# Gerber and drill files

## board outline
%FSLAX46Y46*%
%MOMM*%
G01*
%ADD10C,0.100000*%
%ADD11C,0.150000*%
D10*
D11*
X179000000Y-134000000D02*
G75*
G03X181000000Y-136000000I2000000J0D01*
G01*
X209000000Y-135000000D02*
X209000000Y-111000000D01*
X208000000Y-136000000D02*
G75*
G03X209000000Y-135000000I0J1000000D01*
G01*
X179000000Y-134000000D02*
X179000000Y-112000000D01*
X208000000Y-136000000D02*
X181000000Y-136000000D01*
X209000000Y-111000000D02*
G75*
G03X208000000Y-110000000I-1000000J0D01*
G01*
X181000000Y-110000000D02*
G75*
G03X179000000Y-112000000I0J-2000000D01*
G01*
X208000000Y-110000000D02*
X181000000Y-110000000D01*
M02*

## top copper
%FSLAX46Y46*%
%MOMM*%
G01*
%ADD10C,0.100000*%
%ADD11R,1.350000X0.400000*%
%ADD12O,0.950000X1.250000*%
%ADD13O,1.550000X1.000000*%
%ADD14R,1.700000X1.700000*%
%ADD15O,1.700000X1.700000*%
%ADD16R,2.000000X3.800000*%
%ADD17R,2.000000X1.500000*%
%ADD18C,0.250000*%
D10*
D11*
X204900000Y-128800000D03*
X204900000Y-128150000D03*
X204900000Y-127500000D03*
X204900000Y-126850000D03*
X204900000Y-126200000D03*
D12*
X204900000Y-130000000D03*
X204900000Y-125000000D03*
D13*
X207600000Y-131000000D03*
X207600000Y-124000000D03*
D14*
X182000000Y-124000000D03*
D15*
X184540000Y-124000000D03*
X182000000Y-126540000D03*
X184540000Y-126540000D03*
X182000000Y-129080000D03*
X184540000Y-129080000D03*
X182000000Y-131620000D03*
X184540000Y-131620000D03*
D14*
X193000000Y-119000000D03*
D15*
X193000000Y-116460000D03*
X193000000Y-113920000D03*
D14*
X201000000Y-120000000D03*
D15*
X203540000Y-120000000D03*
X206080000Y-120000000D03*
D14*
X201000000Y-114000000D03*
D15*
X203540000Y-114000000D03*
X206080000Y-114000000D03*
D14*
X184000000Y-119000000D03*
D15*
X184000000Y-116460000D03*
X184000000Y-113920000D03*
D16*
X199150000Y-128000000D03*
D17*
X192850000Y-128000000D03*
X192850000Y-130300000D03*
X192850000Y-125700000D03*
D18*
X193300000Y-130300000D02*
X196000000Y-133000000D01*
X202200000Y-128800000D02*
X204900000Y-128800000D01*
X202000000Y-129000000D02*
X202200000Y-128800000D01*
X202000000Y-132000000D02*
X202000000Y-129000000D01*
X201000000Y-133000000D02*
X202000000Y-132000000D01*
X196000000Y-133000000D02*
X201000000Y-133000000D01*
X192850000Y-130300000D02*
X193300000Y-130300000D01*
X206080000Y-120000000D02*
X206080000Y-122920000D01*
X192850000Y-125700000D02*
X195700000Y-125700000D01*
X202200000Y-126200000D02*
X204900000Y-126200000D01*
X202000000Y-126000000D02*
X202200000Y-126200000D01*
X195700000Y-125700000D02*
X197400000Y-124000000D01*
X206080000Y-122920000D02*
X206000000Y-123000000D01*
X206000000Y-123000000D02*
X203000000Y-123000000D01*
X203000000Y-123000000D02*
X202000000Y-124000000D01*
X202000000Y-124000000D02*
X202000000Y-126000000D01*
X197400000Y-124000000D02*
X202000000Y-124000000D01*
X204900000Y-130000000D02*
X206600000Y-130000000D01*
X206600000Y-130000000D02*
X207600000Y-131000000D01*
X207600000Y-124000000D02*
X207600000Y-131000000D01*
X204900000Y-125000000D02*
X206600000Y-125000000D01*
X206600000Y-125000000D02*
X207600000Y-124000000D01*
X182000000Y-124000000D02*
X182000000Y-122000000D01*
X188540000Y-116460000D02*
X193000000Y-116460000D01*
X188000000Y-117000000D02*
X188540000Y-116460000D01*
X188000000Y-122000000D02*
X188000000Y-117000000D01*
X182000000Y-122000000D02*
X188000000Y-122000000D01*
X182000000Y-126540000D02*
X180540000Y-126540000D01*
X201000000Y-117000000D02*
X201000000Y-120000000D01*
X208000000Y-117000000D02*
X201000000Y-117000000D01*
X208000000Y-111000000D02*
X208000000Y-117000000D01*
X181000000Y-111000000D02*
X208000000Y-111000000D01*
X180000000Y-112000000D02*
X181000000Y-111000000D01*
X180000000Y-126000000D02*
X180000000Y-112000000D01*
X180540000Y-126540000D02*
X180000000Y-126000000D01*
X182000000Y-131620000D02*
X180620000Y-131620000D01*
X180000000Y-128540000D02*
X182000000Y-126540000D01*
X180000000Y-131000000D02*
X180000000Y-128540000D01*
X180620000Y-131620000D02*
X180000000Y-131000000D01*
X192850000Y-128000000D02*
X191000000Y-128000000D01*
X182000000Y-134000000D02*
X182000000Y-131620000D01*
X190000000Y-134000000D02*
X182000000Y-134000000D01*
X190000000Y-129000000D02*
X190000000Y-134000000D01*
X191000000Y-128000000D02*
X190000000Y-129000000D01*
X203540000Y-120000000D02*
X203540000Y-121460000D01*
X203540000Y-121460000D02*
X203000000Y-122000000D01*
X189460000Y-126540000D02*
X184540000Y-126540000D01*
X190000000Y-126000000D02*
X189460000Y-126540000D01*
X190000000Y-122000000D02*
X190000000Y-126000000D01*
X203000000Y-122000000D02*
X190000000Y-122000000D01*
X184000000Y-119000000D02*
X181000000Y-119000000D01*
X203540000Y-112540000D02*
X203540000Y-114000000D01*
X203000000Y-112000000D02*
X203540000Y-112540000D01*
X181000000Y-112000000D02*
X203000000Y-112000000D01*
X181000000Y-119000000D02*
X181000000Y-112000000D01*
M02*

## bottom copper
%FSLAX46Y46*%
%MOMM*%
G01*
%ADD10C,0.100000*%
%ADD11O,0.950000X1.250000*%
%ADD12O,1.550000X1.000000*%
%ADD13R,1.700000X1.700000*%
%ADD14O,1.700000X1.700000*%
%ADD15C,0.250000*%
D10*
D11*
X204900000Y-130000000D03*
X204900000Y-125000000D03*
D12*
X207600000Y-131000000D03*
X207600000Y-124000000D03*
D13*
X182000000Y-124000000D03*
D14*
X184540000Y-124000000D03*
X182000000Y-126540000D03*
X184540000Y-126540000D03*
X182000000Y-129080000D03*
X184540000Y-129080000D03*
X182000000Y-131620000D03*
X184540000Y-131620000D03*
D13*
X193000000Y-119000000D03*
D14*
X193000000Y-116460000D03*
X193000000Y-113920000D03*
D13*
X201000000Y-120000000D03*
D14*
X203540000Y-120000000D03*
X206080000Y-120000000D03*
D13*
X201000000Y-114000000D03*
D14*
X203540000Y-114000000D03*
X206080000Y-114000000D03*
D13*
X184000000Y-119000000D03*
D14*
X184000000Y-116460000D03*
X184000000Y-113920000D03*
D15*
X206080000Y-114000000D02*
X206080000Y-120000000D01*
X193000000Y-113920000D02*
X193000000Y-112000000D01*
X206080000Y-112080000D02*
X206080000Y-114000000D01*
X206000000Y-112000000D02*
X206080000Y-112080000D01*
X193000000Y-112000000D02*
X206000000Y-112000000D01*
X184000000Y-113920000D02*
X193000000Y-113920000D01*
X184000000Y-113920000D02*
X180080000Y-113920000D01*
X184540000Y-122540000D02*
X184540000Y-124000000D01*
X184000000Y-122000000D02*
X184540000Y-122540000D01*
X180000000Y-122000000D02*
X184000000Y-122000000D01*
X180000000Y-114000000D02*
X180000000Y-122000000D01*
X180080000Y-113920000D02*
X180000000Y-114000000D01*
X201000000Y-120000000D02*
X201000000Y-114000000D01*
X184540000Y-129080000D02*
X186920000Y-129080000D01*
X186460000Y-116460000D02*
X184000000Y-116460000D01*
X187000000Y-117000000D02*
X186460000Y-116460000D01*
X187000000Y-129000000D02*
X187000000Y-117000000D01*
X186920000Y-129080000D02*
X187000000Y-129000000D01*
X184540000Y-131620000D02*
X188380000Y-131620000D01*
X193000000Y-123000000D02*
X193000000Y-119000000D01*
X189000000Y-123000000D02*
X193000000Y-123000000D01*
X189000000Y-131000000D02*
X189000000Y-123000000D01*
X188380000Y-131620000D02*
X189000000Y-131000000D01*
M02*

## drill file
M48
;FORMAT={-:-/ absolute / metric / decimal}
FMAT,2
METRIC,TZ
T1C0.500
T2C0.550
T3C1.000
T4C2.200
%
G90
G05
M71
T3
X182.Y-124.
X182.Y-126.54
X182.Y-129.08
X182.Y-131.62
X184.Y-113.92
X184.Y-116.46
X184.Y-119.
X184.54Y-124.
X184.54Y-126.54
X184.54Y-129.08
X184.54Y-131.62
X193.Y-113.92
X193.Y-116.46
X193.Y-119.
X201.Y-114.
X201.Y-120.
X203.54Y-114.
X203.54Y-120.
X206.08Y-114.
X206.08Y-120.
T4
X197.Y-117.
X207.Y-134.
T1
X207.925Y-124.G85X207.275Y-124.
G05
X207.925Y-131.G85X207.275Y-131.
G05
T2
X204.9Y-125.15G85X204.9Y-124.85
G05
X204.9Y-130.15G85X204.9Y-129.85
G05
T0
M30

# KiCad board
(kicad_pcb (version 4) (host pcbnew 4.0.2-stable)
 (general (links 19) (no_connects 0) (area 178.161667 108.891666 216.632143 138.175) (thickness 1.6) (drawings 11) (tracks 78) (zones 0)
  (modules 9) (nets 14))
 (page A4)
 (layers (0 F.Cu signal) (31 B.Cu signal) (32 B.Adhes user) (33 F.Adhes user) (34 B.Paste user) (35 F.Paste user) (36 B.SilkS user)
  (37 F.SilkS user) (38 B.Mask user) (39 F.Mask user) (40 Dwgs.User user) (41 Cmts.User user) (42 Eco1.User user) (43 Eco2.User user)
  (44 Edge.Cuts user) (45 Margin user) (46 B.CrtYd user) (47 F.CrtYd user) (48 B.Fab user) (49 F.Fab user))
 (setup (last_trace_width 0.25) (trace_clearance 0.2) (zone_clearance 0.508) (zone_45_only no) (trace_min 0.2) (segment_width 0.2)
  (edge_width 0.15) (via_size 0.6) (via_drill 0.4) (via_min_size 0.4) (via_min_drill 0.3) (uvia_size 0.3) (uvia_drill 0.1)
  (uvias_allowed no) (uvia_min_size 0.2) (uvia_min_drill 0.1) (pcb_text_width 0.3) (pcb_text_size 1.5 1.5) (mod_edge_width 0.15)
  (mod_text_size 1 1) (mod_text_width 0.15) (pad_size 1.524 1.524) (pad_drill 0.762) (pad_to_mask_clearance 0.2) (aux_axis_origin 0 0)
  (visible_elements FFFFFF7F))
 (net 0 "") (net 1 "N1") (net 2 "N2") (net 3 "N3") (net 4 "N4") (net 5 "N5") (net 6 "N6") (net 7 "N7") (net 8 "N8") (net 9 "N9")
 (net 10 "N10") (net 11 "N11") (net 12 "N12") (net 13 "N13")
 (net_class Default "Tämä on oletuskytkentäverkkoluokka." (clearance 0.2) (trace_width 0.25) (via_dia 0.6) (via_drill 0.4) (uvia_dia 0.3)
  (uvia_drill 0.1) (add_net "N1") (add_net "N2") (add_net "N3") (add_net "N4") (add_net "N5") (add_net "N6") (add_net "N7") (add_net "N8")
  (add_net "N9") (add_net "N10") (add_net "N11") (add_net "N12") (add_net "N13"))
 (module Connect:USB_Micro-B (layer F.Cu) (at 206.25 127.5 90)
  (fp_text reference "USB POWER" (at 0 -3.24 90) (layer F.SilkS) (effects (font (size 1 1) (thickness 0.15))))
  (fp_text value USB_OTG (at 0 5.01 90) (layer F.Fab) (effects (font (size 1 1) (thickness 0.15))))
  (pad 1 smd rect (at -1.3 -1.35 180) (size 1.35 0.4) (layers F.Cu F.Paste F.Mask) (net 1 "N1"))
  (pad 2 smd rect (at -0.65 -1.35 180) (size 1.35 0.4) (layers F.Cu F.Paste F.Mask) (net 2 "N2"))
  (pad 3 smd rect (at 0 -1.35 180) (size 1.35 0.4) (layers F.Cu F.Paste F.Mask) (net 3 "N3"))
  (pad 4 smd rect (at 0.65 -1.35 180) (size 1.35 0.4) (layers F.Cu F.Paste F.Mask) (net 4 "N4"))
  (pad 5 smd rect (at 1.3 -1.35 180) (size 1.35 0.4) (layers F.Cu F.Paste F.Mask) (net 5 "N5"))
  (pad 6 thru_hole oval (at -2.5 -1.35 180) (size 0.95 1.25) (drill oval 0.55 0.85) (layers *.Cu *.Mask) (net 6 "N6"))
  (pad 6 thru_hole oval (at 2.5 -1.35 180) (size 0.95 1.25) (drill oval 0.55 0.85) (layers *.Cu *.Mask) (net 6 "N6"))
  (pad 6 thru_hole oval (at -3.5 1.35 180) (size 1.55 1) (drill oval 1.15 0.5) (layers *.Cu *.Mask) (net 6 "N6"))
  (pad 6 thru_hole oval (at 3.5 1.35 180) (size 1.55 1) (drill oval 1.15 0.5) (layers *.Cu *.Mask) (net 6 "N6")))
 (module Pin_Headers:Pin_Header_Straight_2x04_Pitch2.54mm (layer F.Cu) (at 182 124)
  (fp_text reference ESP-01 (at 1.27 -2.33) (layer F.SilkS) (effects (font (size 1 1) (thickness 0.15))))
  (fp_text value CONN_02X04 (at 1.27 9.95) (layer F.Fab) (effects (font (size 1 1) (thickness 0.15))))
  (pad 1 thru_hole rect (at 0 0) (size 1.7 1.7) (drill 1) (layers *.Cu *.Mask) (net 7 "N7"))
  (pad 2 thru_hole oval (at 2.54 0) (size 1.7 1.7) (drill 1) (layers *.Cu *.Mask) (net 5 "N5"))
  (pad 3 thru_hole oval (at 0 2.54) (size 1.7 1.7) (drill 1) (layers *.Cu *.Mask) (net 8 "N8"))
  (pad 4 thru_hole oval (at 2.54 2.54) (size 1.7 1.7) (drill 1) (layers *.Cu *.Mask) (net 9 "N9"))
  (pad 5 thru_hole oval (at 0 5.08) (size 1.7 1.7) (drill 1) (layers *.Cu *.Mask) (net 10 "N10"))
  (pad 6 thru_hole oval (at 2.54 5.08) (size 1.7 1.7) (drill 1) (layers *.Cu *.Mask) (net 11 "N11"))
  (pad 7 thru_hole oval (at 0 7.62) (size 1.7 1.7) (drill 1) (layers *.Cu *.Mask) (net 8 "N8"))
  (pad 8 thru_hole oval (at 2.54 7.62) (size 1.7 1.7) (drill 1) (layers *.Cu *.Mask) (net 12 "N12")))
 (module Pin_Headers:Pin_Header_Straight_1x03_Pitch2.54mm (layer F.Cu) (at 193 119 180)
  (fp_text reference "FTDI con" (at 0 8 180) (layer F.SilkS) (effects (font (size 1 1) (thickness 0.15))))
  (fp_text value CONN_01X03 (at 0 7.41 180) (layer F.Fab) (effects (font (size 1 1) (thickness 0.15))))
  (pad 1 thru_hole rect (at 0 0 180) (size 1.7 1.7) (drill 1) (layers *.Cu *.Mask) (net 12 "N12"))
  (pad 2 thru_hole oval (at 0 2.54 180) (size 1.7 1.7) (drill 1) (layers *.Cu *.Mask) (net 7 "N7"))
  (pad 3 thru_hole oval (at 0 5.08 180) (size 1.7 1.7) (drill 1) (layers *.Cu *.Mask) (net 5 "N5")))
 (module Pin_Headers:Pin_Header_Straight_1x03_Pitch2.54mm (layer F.Cu) (at 201 120 90)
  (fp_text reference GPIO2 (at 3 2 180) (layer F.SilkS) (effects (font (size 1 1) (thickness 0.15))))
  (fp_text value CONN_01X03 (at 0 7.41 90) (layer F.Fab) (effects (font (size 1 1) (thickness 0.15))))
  (pad 1 thru_hole rect (at 0 0 90) (size 1.7 1.7) (drill 1) (layers *.Cu *.Mask) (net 8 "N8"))
  (pad 2 thru_hole oval (at 0 2.54 90) (size 1.7 1.7) (drill 1) (layers *.Cu *.Mask) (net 9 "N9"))
  (pad 3 thru_hole oval (at 0 5.08 90) (size 1.7 1.7) (drill 1) (layers *.Cu *.Mask) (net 5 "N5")))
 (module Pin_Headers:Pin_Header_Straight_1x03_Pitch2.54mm (layer F.Cu) (at 201 114 90)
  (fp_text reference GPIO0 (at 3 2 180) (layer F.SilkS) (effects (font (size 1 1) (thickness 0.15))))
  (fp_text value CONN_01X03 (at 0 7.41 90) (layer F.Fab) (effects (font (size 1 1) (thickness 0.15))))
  (pad 1 thru_hole rect (at 0 0 90) (size 1.7 1.7) (drill 1) (layers *.Cu *.Mask) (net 8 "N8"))
  (pad 2 thru_hole oval (at 0 2.54 90) (size 1.7 1.7) (drill 1) (layers *.Cu *.Mask) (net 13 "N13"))
  (pad 3 thru_hole oval (at 0 5.08 90) (size 1.7 1.7) (drill 1) (layers *.Cu *.Mask) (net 5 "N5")))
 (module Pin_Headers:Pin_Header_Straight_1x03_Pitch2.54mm (layer F.Cu) (at 184 119 180)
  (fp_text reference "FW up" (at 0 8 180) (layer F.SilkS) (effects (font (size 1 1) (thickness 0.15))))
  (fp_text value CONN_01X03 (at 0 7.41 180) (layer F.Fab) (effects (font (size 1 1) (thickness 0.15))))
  (pad 1 thru_hole rect (at 0 0 180) (size 1.7 1.7) (drill 1) (layers *.Cu *.Mask) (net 13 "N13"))
  (pad 2 thru_hole oval (at 0 2.54 180) (size 1.7 1.7) (drill 1) (layers *.Cu *.Mask) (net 11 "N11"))
  (pad 3 thru_hole oval (at 0 5.08 180) (size 1.7 1.7) (drill 1) (layers *.Cu *.Mask) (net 5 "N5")))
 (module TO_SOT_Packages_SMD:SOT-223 (layer F.Cu) (at 196 128)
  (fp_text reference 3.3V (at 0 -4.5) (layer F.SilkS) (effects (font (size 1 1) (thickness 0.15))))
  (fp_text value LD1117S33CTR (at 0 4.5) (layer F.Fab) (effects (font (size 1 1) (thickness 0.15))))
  (pad 4 smd rect (at 3.15 0) (size 2 3.8) (layers F.Cu F.Paste F.Mask))
  (pad 2 smd rect (at -3.15 0) (size 2 1.5) (layers F.Cu F.Paste F.Mask) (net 8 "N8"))
  (pad 3 smd rect (at -3.15 2.3) (size 2 1.5) (layers F.Cu F.Paste F.Mask) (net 1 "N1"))
  (pad 1 smd rect (at -3.15 -2.3) (size 2 1.5) (layers F.Cu F.Paste F.Mask) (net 5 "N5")))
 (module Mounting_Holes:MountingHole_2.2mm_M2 (layer F.Cu) (at 197 117)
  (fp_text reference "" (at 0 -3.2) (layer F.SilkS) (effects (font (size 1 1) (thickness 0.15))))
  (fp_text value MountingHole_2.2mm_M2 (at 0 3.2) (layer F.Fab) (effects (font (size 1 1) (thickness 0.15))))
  (pad 1 np_thru_hole circle (at 0 0) (size 2.2 2.2) (drill 2.2) (layers *.Cu *.Mask)))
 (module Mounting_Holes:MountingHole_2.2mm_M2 (layer F.Cu) (at 207 134)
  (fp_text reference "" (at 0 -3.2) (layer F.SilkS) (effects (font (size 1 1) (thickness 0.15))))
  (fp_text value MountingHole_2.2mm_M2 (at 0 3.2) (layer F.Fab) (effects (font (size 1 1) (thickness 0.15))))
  (pad 1 np_thru_hole circle (at 0 0) (size 2.2 2.2) (drill 2.2) (layers *.Cu *.Mask)))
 (gr_arc (start 181 134) (end 181 136) (angle 90) (layer Edge.Cuts) (width 0.15))
 (gr_line (start 209 135) (end 209 111) (angle 90) (layer Edge.Cuts) (width 0.15))
 (gr_arc (start 208 135) (end 209 135) (angle 90) (layer Edge.Cuts) (width 0.15))
 (gr_line (start 179 134) (end 179 112) (angle 90) (layer Edge.Cuts) (width 0.15))
 (gr_line (start 208 136) (end 181 136) (angle 90) (layer Edge.Cuts) (width 0.15))
 (gr_arc (start 208 111) (end 208 110) (angle 90) (layer Edge.Cuts) (width 0.15))
 (gr_arc (start 181 112) (end 179 112) (angle 90) (layer Edge.Cuts) (width 0.15))
 (gr_line (start 208 110) (end 181 110) (angle 90) (layer Edge.Cuts) (width 0.15))
 (segment (start 193.3 130.3) (end 196 133) (width 0.25) (layer F.Cu) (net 1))
 (segment (start 202.2 128.8) (end 204.9 128.8) (width 0.25) (layer F.Cu) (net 1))
 (segment (start 202 129) (end 202.2 128.8) (width 0.25) (layer F.Cu) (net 1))
 (segment (start 202 132) (end 202 129) (width 0.25) (layer F.Cu) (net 1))
 (segment (start 201 133) (end 202 132) (width 0.25) (layer F.Cu) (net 1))
 (segment (start 196 133) (end 201 133) (width 0.25) (layer F.Cu) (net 1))
 (segment (start 192.85 130.3) (end 193.3 130.3) (width 0.25) (layer F.Cu) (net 1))
 (segment (start 206.08 114) (end 206.08 120) (width 0.25) (layer B.Cu) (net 5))
 (segment (start 193 113.92) (end 193 112) (width 0.25) (layer B.Cu) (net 5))
 (segment (start 206.08 112.08) (end 206.08 114) (width 0.25) (layer B.Cu) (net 5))
 (segment (start 206 112) (end 206.08 112.08) (width 0.25) (layer B.Cu) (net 5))
 (segment (start 193 112) (end 206 112) (width 0.25) (layer B.Cu) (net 5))
 (segment (start 184 113.92) (end 193 113.92) (width 0.25) (layer B.Cu) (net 5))
 (segment (start 184 113.92) (end 180.08 113.92) (width 0.25) (layer B.Cu) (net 5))
 (segment (start 184.54 122.54) (end 184.54 124) (width 0.25) (layer B.Cu) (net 5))
 (segment (start 184 122) (end 184.54 122.54) (width 0.25) (layer B.Cu) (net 5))
 (segment (start 180 122) (end 184 122) (width 0.25) (layer B.Cu) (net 5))
 (segment (start 180 114) (end 180 122) (width 0.25) (layer B.Cu) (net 5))
 (segment (start 180.08 113.92) (end 180 114) (width 0.25) (layer B.Cu) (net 5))
 (segment (start 206.08 120) (end 206.08 122.92) (width 0.25) (layer F.Cu) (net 5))
 (segment (start 192.85 125.7) (end 195.7 125.7) (width 0.25) (layer F.Cu) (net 5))
 (segment (start 202.2 126.2) (end 204.9 126.2) (width 0.25) (layer F.Cu) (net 5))
 (segment (start 202 126) (end 202.2 126.2) (width 0.25) (layer F.Cu) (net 5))
 (segment (start 195.7 125.7) (end 197.4 124) (width 0.25) (layer F.Cu) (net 5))
 (segment (start 206.08 122.92) (end 206 123) (width 0.25) (layer F.Cu) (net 5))
 (segment (start 206 123) (end 203 123) (width 0.25) (layer F.Cu) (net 5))
 (segment (start 203 123) (end 202 124) (width 0.25) (layer F.Cu) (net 5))
 (segment (start 202 124) (end 202 126) (width 0.25) (layer F.Cu) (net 5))
 (segment (start 197.4 124) (end 202 124) (width 0.25) (layer F.Cu) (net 5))
 (segment (start 204.9 130) (end 206.6 130) (width 0.25) (layer F.Cu) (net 6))
 (segment (start 206.6 130) (end 207.6 131) (width 0.25) (layer F.Cu) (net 6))
 (segment (start 207.6 124) (end 207.6 131) (width 0.25) (layer F.Cu) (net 6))
 (segment (start 204.9 125) (end 206.6 125) (width 0.25) (layer F.Cu) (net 6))
 (segment (start 206.6 125) (end 207.6 124) (width 0.25) (layer F.Cu) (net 6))
 (segment (start 182 124) (end 182 122) (width 0.25) (layer F.Cu) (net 7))
 (segment (start 188.54 116.46) (end 193 116.46) (width 0.25) (layer F.Cu) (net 7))
 (segment (start 188 117) (end 188.54 116.46) (width 0.25) (layer F.Cu) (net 7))
 (segment (start 188 122) (end 188 117) (width 0.25) (layer F.Cu) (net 7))
 (segment (start 182 122) (end 188 122) (width 0.25) (layer F.Cu) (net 7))
 (segment (start 201 120) (end 201 114) (width 0.25) (layer B.Cu) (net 8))
 (segment (start 182 126.54) (end 180.54 126.54) (width 0.25) (layer F.Cu) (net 8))
 (segment (start 201 117) (end 201 120) (width 0.25) (layer F.Cu) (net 8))
 (segment (start 208 117) (end 201 117) (width 0.25) (layer F.Cu) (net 8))
 (segment (start 208 111) (end 208 117) (width 0.25) (layer F.Cu) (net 8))
 (segment (start 181 111) (end 208 111) (width 0.25) (layer F.Cu) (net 8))
 (segment (start 180 112) (end 181 111) (width 0.25) (layer F.Cu) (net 8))
 (segment (start 180 126) (end 180 112) (width 0.25) (layer F.Cu) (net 8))
 (segment (start 180.54 126.54) (end 180 126) (width 0.25) (layer F.Cu) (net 8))
 (segment (start 182 131.62) (end 180.62 131.62) (width 0.25) (layer F.Cu) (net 8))
 (segment (start 180 128.54) (end 182 126.54) (width 0.25) (layer F.Cu) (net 8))
 (segment (start 180 131) (end 180 128.54) (width 0.25) (layer F.Cu) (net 8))
 (segment (start 180.62 131.62) (end 180 131) (width 0.25) (layer F.Cu) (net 8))
 (segment (start 192.85 128) (end 191 128) (width 0.25) (layer F.Cu) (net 8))
 (segment (start 182 134) (end 182 131.62) (width 0.25) (layer F.Cu) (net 8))
 (segment (start 190 134) (end 182 134) (width 0.25) (layer F.Cu) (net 8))
 (segment (start 190 129) (end 190 134) (width 0.25) (layer F.Cu) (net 8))
 (segment (start 191 128) (end 190 129) (width 0.25) (layer F.Cu) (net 8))
 (segment (start 203.54 120) (end 203.54 121.46) (width 0.25) (layer F.Cu) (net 9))
 (segment (start 203.54 121.46) (end 203 122) (width 0.25) (layer F.Cu) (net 9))
 (segment (start 189.46 126.54) (end 184.54 126.54) (width 0.25) (layer F.Cu) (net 9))
 (segment (start 190 126) (end 189.46 126.54) (width 0.25) (layer F.Cu) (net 9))
 (segment (start 190 122) (end 190 126) (width 0.25) (layer F.Cu) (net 9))
 (segment (start 203 122) (end 190 122) (width 0.25) (layer F.Cu) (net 9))
 (segment (start 184.54 129.08) (end 186.92 129.08) (width 0.25) (layer B.Cu) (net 11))
 (segment (start 186.46 116.46) (end 184 116.46) (width 0.25) (layer B.Cu) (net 11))
 (segment (start 187 117) (end 186.46 116.46) (width 0.25) (layer B.Cu) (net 11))
 (segment (start 187 129) (end 187 117) (width 0.25) (layer B.Cu) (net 11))
 (segment (start 186.92 129.08) (end 187 129) (width 0.25) (layer B.Cu) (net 11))
 (segment (start 184.54 131.62) (end 188.38 131.62) (width 0.25) (layer B.Cu) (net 12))
 (segment (start 193 123) (end 193 119) (width 0.25) (layer B.Cu) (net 12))
 (segment (start 189 123) (end 193 123) (width 0.25) (layer B.Cu) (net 12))
 (segment (start 189 131) (end 189 123) (width 0.25) (layer B.Cu) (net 12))
 (segment (start 188.38 131.62) (end 189 131) (width 0.25) (layer B.Cu) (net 12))
 (segment (start 184 119) (end 181 119) (width 0.25) (layer F.Cu) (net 13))
 (segment (start 203.54 112.54) (end 203.54 114) (width 0.25) (layer F.Cu) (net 13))
 (segment (start 203 112) (end 203.54 112.54) (width 0.25) (layer F.Cu) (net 13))
 (segment (start 181 112) (end 203 112) (width 0.25) (layer F.Cu) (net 13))
 (segment (start 181 119) (end 181 112) (width 0.25) (layer F.Cu) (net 13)))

